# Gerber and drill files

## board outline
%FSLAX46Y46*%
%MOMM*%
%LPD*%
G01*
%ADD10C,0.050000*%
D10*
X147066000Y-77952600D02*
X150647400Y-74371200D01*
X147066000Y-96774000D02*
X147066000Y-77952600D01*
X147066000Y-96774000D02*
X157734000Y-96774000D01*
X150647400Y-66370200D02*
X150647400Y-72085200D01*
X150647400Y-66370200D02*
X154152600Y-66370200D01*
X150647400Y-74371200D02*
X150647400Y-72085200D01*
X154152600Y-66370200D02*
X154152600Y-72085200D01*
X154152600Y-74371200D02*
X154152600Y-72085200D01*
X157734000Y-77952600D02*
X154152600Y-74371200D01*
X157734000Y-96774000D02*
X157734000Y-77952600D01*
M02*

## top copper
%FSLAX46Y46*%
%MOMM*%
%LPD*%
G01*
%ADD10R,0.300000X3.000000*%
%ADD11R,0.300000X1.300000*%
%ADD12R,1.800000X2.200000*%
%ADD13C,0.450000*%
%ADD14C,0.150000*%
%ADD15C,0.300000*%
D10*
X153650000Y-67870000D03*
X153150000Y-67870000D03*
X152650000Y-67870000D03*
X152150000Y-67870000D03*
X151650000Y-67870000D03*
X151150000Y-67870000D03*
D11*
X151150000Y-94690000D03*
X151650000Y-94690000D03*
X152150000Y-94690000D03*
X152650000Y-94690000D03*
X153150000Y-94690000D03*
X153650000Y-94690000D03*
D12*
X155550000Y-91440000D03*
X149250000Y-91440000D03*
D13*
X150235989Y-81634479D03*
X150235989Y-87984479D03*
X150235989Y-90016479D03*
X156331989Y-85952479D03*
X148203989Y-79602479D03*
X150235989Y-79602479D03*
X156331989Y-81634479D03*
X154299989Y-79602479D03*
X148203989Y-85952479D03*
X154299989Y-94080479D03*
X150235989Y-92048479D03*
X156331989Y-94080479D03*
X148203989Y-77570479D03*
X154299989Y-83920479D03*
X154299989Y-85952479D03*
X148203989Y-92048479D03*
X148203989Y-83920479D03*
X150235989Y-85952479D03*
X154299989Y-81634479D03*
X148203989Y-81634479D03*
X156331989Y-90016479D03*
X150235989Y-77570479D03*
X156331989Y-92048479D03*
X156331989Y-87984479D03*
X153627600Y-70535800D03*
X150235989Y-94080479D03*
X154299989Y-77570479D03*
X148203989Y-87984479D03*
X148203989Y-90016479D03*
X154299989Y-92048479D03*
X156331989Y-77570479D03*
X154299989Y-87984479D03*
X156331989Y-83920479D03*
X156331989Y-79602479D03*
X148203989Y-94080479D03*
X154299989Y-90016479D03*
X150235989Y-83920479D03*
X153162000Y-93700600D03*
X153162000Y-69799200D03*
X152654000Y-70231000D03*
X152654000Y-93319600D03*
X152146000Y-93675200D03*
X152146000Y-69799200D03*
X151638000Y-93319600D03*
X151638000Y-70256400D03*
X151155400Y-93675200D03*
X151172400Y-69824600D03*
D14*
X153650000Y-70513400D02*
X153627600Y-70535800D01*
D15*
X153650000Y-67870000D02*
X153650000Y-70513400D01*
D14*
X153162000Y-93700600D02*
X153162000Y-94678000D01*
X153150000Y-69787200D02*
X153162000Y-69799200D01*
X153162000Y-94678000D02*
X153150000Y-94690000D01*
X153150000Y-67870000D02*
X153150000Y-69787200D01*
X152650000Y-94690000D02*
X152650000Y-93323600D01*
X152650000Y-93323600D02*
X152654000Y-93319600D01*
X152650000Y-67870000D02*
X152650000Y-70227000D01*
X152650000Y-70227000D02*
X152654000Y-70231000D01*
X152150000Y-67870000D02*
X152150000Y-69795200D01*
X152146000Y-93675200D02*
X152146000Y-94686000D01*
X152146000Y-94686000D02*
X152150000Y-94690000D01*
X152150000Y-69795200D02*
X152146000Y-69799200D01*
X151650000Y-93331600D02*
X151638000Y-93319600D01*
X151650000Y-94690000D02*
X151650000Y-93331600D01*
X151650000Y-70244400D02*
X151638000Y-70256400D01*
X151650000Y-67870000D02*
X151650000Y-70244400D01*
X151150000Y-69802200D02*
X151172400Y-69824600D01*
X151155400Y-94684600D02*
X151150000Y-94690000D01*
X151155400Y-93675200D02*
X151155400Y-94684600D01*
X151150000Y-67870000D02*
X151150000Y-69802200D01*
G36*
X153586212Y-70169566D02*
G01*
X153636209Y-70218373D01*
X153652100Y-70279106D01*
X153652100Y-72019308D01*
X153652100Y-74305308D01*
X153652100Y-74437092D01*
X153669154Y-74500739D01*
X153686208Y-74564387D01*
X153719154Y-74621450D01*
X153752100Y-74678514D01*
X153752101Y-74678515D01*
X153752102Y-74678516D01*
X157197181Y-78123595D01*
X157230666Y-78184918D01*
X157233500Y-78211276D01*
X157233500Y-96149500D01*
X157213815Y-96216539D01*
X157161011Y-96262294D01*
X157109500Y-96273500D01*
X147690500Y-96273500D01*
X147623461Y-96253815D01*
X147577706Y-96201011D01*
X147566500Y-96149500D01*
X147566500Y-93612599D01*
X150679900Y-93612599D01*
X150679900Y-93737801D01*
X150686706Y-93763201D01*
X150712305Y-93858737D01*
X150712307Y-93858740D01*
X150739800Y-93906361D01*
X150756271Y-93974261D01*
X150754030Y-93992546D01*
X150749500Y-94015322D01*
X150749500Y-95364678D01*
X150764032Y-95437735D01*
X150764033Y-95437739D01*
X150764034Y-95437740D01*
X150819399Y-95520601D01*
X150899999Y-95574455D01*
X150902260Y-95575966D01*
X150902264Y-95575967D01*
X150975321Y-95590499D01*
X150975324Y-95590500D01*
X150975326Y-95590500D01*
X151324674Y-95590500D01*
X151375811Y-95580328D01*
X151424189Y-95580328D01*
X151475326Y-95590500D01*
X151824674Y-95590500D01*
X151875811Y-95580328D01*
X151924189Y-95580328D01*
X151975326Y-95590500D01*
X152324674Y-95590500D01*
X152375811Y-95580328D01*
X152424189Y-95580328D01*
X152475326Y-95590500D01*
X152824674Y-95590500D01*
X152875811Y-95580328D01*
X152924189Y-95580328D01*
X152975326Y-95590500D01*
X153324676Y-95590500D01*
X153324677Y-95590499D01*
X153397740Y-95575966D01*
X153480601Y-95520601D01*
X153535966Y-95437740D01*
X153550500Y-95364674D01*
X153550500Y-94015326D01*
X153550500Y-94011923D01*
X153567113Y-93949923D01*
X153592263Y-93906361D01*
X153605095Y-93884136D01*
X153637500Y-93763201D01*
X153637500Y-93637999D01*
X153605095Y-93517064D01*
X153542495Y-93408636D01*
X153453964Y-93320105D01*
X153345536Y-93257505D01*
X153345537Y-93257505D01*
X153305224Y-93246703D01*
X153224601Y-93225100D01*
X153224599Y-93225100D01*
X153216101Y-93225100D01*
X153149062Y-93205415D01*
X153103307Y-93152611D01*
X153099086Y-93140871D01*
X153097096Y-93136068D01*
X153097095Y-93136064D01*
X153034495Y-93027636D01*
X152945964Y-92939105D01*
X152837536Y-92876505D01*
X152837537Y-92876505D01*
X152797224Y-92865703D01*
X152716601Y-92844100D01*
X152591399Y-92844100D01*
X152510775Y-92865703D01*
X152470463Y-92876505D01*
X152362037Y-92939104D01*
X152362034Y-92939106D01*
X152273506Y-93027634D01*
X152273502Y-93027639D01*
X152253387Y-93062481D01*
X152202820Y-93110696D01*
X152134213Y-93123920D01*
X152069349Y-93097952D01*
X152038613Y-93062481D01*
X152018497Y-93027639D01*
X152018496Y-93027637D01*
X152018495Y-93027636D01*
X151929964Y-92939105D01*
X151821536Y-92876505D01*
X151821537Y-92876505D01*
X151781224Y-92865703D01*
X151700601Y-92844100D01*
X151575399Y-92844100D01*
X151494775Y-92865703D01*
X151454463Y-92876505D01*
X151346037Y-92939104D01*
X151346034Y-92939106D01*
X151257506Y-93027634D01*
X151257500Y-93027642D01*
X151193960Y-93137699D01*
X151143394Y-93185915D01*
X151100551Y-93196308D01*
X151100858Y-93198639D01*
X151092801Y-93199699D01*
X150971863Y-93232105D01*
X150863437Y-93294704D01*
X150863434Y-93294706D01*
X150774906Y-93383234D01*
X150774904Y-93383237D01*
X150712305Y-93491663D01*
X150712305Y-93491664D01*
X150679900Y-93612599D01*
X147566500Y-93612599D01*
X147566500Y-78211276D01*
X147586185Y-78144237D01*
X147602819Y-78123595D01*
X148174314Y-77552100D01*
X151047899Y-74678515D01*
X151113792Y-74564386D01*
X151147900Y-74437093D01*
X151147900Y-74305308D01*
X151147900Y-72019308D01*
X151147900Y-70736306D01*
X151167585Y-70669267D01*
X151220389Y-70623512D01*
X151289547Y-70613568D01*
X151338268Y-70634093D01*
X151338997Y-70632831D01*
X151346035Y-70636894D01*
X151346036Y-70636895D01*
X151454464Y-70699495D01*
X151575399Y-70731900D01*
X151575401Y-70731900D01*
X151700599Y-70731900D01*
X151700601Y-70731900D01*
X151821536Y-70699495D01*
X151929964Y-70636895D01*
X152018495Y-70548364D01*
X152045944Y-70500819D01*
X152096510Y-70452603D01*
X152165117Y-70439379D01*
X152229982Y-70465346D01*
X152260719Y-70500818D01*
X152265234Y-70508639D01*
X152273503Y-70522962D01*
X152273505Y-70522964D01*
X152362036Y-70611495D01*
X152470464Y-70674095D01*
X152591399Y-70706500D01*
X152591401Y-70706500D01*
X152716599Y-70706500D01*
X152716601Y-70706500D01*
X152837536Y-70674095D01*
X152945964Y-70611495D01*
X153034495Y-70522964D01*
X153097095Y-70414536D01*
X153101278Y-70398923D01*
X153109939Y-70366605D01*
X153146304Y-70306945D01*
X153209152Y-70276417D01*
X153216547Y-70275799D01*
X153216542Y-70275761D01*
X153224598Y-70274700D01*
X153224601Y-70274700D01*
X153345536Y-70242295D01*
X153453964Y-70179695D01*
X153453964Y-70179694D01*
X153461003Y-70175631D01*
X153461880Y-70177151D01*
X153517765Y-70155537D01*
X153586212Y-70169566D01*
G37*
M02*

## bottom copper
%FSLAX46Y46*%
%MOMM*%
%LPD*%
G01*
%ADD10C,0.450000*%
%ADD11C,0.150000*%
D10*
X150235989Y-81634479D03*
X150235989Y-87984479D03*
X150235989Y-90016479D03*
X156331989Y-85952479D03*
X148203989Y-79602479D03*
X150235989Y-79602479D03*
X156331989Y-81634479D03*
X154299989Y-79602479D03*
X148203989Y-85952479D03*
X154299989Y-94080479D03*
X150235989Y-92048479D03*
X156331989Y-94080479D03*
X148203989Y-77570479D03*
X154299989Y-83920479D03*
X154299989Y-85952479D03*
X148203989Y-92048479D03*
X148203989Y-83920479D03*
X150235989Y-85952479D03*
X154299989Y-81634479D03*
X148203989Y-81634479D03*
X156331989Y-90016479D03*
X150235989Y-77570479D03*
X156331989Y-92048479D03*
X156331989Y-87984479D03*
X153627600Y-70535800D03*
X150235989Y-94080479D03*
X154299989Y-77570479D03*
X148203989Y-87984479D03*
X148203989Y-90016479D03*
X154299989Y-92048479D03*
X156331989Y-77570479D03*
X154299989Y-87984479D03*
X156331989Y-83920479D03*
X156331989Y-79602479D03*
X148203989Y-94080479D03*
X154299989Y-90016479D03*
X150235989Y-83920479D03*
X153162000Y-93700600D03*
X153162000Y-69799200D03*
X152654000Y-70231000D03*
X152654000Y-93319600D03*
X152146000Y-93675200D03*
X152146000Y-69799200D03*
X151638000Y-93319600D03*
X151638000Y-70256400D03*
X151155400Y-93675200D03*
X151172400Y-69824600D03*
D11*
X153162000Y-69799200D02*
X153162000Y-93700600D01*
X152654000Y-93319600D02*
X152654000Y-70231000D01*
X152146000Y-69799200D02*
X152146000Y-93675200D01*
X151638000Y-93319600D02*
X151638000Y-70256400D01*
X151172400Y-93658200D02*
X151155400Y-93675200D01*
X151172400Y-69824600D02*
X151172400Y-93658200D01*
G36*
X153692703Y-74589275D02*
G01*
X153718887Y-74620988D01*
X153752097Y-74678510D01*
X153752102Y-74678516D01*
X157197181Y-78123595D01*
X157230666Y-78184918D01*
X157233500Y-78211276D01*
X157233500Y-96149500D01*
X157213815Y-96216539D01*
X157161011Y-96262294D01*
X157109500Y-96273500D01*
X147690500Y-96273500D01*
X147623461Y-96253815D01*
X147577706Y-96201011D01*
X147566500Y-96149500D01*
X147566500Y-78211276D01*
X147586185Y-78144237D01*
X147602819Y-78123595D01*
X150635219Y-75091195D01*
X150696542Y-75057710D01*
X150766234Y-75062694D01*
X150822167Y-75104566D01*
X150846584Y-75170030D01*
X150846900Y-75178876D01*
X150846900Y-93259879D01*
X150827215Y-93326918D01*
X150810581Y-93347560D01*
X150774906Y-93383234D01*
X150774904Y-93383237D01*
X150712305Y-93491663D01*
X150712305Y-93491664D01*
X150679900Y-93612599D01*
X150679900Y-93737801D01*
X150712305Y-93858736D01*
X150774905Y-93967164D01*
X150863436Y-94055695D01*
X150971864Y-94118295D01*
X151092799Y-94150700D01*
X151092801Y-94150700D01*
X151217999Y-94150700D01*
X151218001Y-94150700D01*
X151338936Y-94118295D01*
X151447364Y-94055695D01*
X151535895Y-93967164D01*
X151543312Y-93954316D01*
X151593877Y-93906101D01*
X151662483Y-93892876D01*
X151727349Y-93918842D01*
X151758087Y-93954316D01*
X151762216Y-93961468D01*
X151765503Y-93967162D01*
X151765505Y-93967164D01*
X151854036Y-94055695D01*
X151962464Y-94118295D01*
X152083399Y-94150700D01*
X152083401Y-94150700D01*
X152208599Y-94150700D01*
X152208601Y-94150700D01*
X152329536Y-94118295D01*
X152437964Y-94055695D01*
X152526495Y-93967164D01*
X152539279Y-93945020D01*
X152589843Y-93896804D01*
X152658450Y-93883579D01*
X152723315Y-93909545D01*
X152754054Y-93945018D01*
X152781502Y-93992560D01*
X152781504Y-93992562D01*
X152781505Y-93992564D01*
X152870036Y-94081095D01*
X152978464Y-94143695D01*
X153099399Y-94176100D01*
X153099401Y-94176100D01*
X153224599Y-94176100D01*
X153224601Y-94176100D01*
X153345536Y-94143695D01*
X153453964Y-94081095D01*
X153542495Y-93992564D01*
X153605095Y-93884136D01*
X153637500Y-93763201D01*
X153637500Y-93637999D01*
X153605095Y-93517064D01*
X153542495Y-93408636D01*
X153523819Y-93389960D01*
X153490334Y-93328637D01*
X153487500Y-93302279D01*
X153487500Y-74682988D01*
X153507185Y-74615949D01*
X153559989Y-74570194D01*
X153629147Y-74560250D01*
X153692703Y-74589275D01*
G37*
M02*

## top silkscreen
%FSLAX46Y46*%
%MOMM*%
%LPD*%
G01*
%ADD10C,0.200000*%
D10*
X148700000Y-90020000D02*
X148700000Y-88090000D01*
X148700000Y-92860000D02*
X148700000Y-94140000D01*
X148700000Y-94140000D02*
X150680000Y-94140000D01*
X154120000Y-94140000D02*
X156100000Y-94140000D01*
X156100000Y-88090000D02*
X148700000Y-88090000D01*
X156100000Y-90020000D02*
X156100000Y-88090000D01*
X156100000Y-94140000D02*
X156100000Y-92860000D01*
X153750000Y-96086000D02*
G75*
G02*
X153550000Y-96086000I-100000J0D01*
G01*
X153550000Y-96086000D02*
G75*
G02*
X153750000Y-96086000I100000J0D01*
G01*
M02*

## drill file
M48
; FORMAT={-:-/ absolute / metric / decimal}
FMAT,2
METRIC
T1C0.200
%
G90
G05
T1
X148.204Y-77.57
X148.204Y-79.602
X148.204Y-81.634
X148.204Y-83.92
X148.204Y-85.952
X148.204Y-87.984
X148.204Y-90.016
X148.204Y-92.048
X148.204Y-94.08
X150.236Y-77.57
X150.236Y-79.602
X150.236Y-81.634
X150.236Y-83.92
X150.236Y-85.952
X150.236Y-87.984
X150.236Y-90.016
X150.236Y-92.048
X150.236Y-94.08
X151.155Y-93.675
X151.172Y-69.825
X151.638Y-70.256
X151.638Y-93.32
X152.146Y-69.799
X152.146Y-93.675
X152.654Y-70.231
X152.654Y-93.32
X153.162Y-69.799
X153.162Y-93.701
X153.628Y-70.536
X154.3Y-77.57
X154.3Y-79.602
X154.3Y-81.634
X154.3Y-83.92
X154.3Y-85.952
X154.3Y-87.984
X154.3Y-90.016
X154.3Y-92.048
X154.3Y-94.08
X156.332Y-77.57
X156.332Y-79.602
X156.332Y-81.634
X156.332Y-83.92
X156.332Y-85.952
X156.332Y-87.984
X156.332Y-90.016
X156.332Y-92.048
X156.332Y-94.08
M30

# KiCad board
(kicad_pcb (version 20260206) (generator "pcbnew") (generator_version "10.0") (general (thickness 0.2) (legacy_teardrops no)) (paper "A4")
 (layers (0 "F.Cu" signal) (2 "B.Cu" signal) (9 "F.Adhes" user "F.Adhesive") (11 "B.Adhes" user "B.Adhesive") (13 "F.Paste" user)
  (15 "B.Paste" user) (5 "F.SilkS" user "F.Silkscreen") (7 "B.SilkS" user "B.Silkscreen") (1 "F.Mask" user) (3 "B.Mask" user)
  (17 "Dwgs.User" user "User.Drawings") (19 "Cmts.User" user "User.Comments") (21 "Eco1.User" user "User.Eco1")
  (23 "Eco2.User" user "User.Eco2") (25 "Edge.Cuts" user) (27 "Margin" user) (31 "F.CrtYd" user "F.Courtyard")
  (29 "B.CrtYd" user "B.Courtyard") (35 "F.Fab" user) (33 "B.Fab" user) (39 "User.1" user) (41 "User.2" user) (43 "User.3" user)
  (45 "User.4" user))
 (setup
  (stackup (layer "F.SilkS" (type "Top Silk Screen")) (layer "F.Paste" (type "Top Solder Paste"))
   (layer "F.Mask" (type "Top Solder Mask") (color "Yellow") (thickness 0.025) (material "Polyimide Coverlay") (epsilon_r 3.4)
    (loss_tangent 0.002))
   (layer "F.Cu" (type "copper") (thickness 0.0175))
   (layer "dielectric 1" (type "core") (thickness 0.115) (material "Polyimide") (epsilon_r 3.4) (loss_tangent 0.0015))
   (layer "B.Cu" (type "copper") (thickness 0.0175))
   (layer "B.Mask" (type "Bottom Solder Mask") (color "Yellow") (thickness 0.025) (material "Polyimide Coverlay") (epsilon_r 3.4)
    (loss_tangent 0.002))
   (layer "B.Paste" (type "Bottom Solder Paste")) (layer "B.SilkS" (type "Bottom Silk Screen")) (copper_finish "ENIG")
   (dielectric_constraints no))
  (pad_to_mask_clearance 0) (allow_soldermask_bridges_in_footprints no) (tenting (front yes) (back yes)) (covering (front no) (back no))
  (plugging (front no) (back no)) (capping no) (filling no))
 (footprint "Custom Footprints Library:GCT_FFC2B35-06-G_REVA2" (layer "F.Cu") (at 152.4 71.12)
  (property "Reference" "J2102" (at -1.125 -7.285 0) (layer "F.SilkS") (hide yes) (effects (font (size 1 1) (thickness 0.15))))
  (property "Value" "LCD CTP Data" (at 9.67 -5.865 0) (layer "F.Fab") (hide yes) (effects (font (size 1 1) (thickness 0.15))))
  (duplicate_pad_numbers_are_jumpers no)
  (pad "1" smd rect (at 1.25 -3.25) (size 0.3 3) (layers "F.Cu" "F.Mask" "F.Paste") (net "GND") (solder_mask_margin 0.102))
  (pad "2" smd rect (at 0.75 -3.25) (size 0.3 3) (layers "F.Cu" "F.Mask" "F.Paste") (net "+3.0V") (solder_mask_margin 0.102))
  (pad "3" smd rect (at 0.25 -3.25) (size 0.3 3) (layers "F.Cu" "F.Mask" "F.Paste") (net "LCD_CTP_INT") (solder_mask_margin 0.102))
  (pad "4" smd rect (at -0.25 -3.25) (size 0.3 3) (layers "F.Cu" "F.Mask" "F.Paste") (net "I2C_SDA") (solder_mask_margin 0.102))
  (pad "5" smd rect (at -0.75 -3.25) (size 0.3 3) (layers "F.Cu" "F.Mask" "F.Paste") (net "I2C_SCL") (solder_mask_margin 0.102))
  (pad "6" smd rect (at -1.25 -3.25) (size 0.3 3) (layers "F.Cu" "F.Mask" "F.Paste") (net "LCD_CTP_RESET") (solder_mask_margin 0.102)))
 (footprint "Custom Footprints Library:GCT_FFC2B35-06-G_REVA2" (layer "F.Cu") (at 152.4 91.44 180)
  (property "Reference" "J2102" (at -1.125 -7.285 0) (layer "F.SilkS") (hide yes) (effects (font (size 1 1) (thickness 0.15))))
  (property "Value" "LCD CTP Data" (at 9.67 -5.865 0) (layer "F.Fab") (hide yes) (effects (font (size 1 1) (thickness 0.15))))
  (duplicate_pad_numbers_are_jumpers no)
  (fp_line (start 3.7 1.42) (end 3.7 3.35) (stroke (width 0.2) (type solid)) (layer "F.SilkS"))
  (fp_line (start 3.7 -1.42) (end 3.7 -2.7) (stroke (width 0.2) (type solid)) (layer "F.SilkS"))
  (fp_line (start 3.7 -2.7) (end 1.72 -2.7) (stroke (width 0.2) (type solid)) (layer "F.SilkS"))
  (fp_line (start -1.72 -2.7) (end -3.7 -2.7) (stroke (width 0.2) (type solid)) (layer "F.SilkS"))
  (fp_line (start -3.7 3.35) (end 3.7 3.35) (stroke (width 0.2) (type solid)) (layer "F.SilkS"))
  (fp_line (start -3.7 1.42) (end -3.7 3.35) (stroke (width 0.2) (type solid)) (layer "F.SilkS"))
  (fp_line (start -3.7 -2.7) (end -3.7 -1.42) (stroke (width 0.2) (type solid)) (layer "F.SilkS"))
  (fp_circle (center -1.25 -4.646) (end -1.15 -4.646) (stroke (width 0.2) (type solid)) (fill no) (layer "F.SilkS"))
  (pad "1" smd rect (at 1.25 -3.25 180) (size 0.3 1.3) (layers "F.Cu" "F.Mask" "F.Paste") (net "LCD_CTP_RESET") (solder_mask_margin 0.102))
  (pad "2" smd rect (at 0.75 -3.25 180) (size 0.3 1.3) (layers "F.Cu" "F.Mask" "F.Paste") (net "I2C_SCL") (solder_mask_margin 0.102))
  (pad "3" smd rect (at 0.25 -3.25 180) (size 0.3 1.3) (layers "F.Cu" "F.Mask" "F.Paste") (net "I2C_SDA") (solder_mask_margin 0.102))
  (pad "4" smd rect (at -0.25 -3.25 180) (size 0.3 1.3) (layers "F.Cu" "F.Mask" "F.Paste") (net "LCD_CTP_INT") (solder_mask_margin 0.102))
  (pad "5" smd rect (at -0.75 -3.25 180) (size 0.3 1.3) (layers "F.Cu" "F.Mask" "F.Paste") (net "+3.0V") (solder_mask_margin 0.102))
  (pad "6" smd rect (at -1.25 -3.25 180) (size 0.3 1.3) (layers "F.Cu" "F.Mask" "F.Paste") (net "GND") (solder_mask_margin 0.102)
   (zone_connect 2))
  (pad "S1" smd rect (at -3.15 0 180) (size 1.8 2.2) (layers "F.Cu" "F.Mask" "F.Paste") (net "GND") (solder_mask_margin 0.102))
  (pad "S2" smd rect (at 3.15 0 180) (size 1.8 2.2) (layers "F.Cu" "F.Mask" "F.Paste") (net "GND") (solder_mask_margin 0.102)))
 (gr_line (start 147.066 77.9526) (end 150.6474 74.3712) (stroke (width 0.05) (type default)) (layer "Edge.Cuts"))
 (gr_line (start 147.066 96.774) (end 147.066 77.9526) (stroke (width 0.05) (type default)) (layer "Edge.Cuts"))
 (gr_line (start 147.066 96.774) (end 157.734 96.774) (stroke (width 0.05) (type default)) (layer "Edge.Cuts"))
 (gr_line (start 150.6474 66.3702) (end 150.6474 72.0852) (stroke (width 0.05) (type default)) (layer "Edge.Cuts"))
 (gr_line (start 150.6474 66.3702) (end 154.1526 66.3702) (stroke (width 0.05) (type default)) (layer "Edge.Cuts"))
 (gr_line (start 150.6474 74.3712) (end 150.6474 72.0852) (stroke (width 0.05) (type default)) (layer "Edge.Cuts"))
 (gr_line (start 154.1526 66.3702) (end 154.1526 72.0852) (stroke (width 0.05) (type default)) (layer "Edge.Cuts"))
 (gr_line (start 154.1526 74.3712) (end 154.1526 72.0852) (stroke (width 0.05) (type default)) (layer "Edge.Cuts"))
 (gr_line (start 157.734 77.9526) (end 154.1526 74.3712) (stroke (width 0.05) (type default)) (layer "Edge.Cuts"))
 (gr_line (start 157.734 96.774) (end 157.734 77.9526) (stroke (width 0.05) (type default)) (layer "Edge.Cuts"))
 (segment (start 153.65 70.5134) (end 153.6276 70.5358) (width 0.15) (layer "F.Cu") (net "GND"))
 (segment (start 153.65 67.87) (end 153.65 70.5134) (width 0.3) (layer "F.Cu") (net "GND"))
 (via (at 150.235989 81.634479) (size 0.45) (drill 0.2) (layers "F.Cu" "B.Cu") (free yes) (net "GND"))
 (via (at 150.235989 87.984479) (size 0.45) (drill 0.2) (layers "F.Cu" "B.Cu") (free yes) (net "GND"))
 (via (at 150.235989 90.016479) (size 0.45) (drill 0.2) (layers "F.Cu" "B.Cu") (free yes) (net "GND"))
 (via (at 156.331989 85.952479) (size 0.45) (drill 0.2) (layers "F.Cu" "B.Cu") (free yes) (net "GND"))
 (via (at 148.203989 79.602479) (size 0.45) (drill 0.2) (layers "F.Cu" "B.Cu") (free yes) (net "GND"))
 (via (at 150.235989 79.602479) (size 0.45) (drill 0.2) (layers "F.Cu" "B.Cu") (free yes) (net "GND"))
 (via (at 156.331989 81.634479) (size 0.45) (drill 0.2) (layers "F.Cu" "B.Cu") (free yes) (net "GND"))
 (via (at 154.299989 79.602479) (size 0.45) (drill 0.2) (layers "F.Cu" "B.Cu") (free yes) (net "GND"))
 (via (at 148.203989 85.952479) (size 0.45) (drill 0.2) (layers "F.Cu" "B.Cu") (free yes) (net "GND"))
 (via (at 154.299989 94.080479) (size 0.45) (drill 0.2) (layers "F.Cu" "B.Cu") (free yes) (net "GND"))
 (via (at 150.235989 92.048479) (size 0.45) (drill 0.2) (layers "F.Cu" "B.Cu") (free yes) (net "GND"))
 (via (at 156.331989 94.080479) (size 0.45) (drill 0.2) (layers "F.Cu" "B.Cu") (free yes) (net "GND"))
 (via (at 148.203989 77.570479) (size 0.45) (drill 0.2) (layers "F.Cu" "B.Cu") (free yes) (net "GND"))
 (via (at 154.299989 83.920479) (size 0.45) (drill 0.2) (layers "F.Cu" "B.Cu") (free yes) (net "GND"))
 (via (at 154.299989 85.952479) (size 0.45) (drill 0.2) (layers "F.Cu" "B.Cu") (free yes) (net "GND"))
 (via (at 148.203989 92.048479) (size 0.45) (drill 0.2) (layers "F.Cu" "B.Cu") (free yes) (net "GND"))
 (via (at 148.203989 83.920479) (size 0.45) (drill 0.2) (layers "F.Cu" "B.Cu") (free yes) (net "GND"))
 (via (at 150.235989 85.952479) (size 0.45) (drill 0.2) (layers "F.Cu" "B.Cu") (free yes) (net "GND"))
 (via (at 154.299989 81.634479) (size 0.45) (drill 0.2) (layers "F.Cu" "B.Cu") (free yes) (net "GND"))
 (via (at 148.203989 81.634479) (size 0.45) (drill 0.2) (layers "F.Cu" "B.Cu") (free yes) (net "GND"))
 (via (at 156.331989 90.016479) (size 0.45) (drill 0.2) (layers "F.Cu" "B.Cu") (free yes) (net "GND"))
 (via (at 150.235989 77.570479) (size 0.45) (drill 0.2) (layers "F.Cu" "B.Cu") (free yes) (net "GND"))
 (via (at 156.331989 92.048479) (size 0.45) (drill 0.2) (layers "F.Cu" "B.Cu") (free yes) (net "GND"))
 (via (at 156.331989 87.984479) (size 0.45) (drill 0.2) (layers "F.Cu" "B.Cu") (free yes) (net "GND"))
 (via (at 153.6276 70.5358) (size 0.45) (drill 0.2) (layers "F.Cu" "B.Cu") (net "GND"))
 (via (at 150.235989 94.080479) (size 0.45) (drill 0.2) (layers "F.Cu" "B.Cu") (free yes) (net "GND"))
 (via (at 154.299989 77.570479) (size 0.45) (drill 0.2) (layers "F.Cu" "B.Cu") (free yes) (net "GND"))
 (via (at 148.203989 87.984479) (size 0.45) (drill 0.2) (layers "F.Cu" "B.Cu") (free yes) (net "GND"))
 (via (at 148.203989 90.016479) (size 0.45) (drill 0.2) (layers "F.Cu" "B.Cu") (free yes) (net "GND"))
 (via (at 154.299989 92.048479) (size 0.45) (drill 0.2) (layers "F.Cu" "B.Cu") (free yes) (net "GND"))
 (via (at 156.331989 77.570479) (size 0.45) (drill 0.2) (layers "F.Cu" "B.Cu") (free yes) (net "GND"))
 (via (at 154.299989 87.984479) (size 0.45) (drill 0.2) (layers "F.Cu" "B.Cu") (free yes) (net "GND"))
 (via (at 156.331989 83.920479) (size 0.45) (drill 0.2) (layers "F.Cu" "B.Cu") (free yes) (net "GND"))
 (via (at 156.331989 79.602479) (size 0.45) (drill 0.2) (layers "F.Cu" "B.Cu") (free yes) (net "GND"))
 (via (at 148.203989 94.080479) (size 0.45) (drill 0.2) (layers "F.Cu" "B.Cu") (free yes) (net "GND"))
 (via (at 154.299989 90.016479) (size 0.45) (drill 0.2) (layers "F.Cu" "B.Cu") (free yes) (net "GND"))
 (via (at 150.235989 83.920479) (size 0.45) (drill 0.2) (layers "F.Cu" "B.Cu") (free yes) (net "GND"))
 (segment (start 153.162 93.7006) (end 153.162 94.678) (width 0.15) (layer "F.Cu") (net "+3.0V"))
 (segment (start 153.15 69.7872) (end 153.162 69.7992) (width 0.15) (layer "F.Cu") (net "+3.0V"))
 (segment (start 153.162 94.678) (end 153.15 94.69) (width 0.15) (layer "F.Cu") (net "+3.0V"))
 (segment (start 153.15 67.87) (end 153.15 69.7872) (width 0.15) (layer "F.Cu") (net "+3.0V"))
 (via (at 153.162 93.7006) (size 0.45) (drill 0.2) (layers "F.Cu" "B.Cu") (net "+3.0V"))
 (via (at 153.162 69.7992) (size 0.45) (drill 0.2) (layers "F.Cu" "B.Cu") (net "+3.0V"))
 (segment (start 153.162 69.7992) (end 153.162 93.7006) (width 0.15) (layer "B.Cu") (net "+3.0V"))
 (segment (start 152.65 94.69) (end 152.65 93.3236) (width 0.15) (layer "F.Cu") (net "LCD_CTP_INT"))
 (segment (start 152.65 93.3236) (end 152.654 93.3196) (width 0.15) (layer "F.Cu") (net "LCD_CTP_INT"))
 (segment (start 152.65 67.87) (end 152.65 70.227) (width 0.15) (layer "F.Cu") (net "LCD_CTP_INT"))
 (segment (start 152.65 70.227) (end 152.654 70.231) (width 0.15) (layer "F.Cu") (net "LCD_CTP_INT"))
 (via (at 152.654 70.231) (size 0.45) (drill 0.2) (layers "F.Cu" "B.Cu") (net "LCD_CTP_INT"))
 (via (at 152.654 93.3196) (size 0.45) (drill 0.2) (layers "F.Cu" "B.Cu") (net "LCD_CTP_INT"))
 (segment (start 152.654 93.3196) (end 152.654 70.231) (width 0.15) (layer "B.Cu") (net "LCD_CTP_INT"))
 (segment (start 152.15 67.87) (end 152.15 69.7952) (width 0.15) (layer "F.Cu") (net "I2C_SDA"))
 (segment (start 152.146 93.6752) (end 152.146 94.686) (width 0.15) (layer "F.Cu") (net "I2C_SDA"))
 (segment (start 152.146 94.686) (end 152.15 94.69) (width 0.15) (layer "F.Cu") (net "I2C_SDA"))
 (segment (start 152.15 69.7952) (end 152.146 69.7992) (width 0.15) (layer "F.Cu") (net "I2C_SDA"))
 (via (at 152.146 93.6752) (size 0.45) (drill 0.2) (layers "F.Cu" "B.Cu") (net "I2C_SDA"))
 (via (at 152.146 69.7992) (size 0.45) (drill 0.2) (layers "F.Cu" "B.Cu") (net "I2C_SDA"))
 (segment (start 152.146 69.7992) (end 152.146 93.6752) (width 0.15) (layer "B.Cu") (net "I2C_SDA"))
 (segment (start 151.65 93.3316) (end 151.638 93.3196) (width 0.15) (layer "F.Cu") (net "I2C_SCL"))
 (segment (start 151.65 94.69) (end 151.65 93.3316) (width 0.15) (layer "F.Cu") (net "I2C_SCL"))
 (segment (start 151.65 70.2444) (end 151.638 70.2564) (width 0.15) (layer "F.Cu") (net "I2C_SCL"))
 (segment (start 151.65 67.87) (end 151.65 70.2444) (width 0.15) (layer "F.Cu") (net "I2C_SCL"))
 (via (at 151.638 93.3196) (size 0.45) (drill 0.2) (layers "F.Cu" "B.Cu") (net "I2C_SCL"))
 (via (at 151.638 70.2564) (size 0.45) (drill 0.2) (layers "F.Cu" "B.Cu") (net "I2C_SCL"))
 (segment (start 151.638 93.3196) (end 151.638 70.2564) (width 0.15) (layer "B.Cu") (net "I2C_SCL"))
 (segment (start 151.15 69.8022) (end 151.1724 69.8246) (width 0.15) (layer "F.Cu") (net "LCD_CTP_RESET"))
 (segment (start 151.1554 94.6846) (end 151.15 94.69) (width 0.15) (layer "F.Cu") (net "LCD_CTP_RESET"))
 (segment (start 151.1554 93.6752) (end 151.1554 94.6846) (width 0.15) (layer "F.Cu") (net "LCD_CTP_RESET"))
 (segment (start 151.15 67.87) (end 151.15 69.8022) (width 0.15) (layer "F.Cu") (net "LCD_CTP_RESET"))
 (via (at 151.1554 93.6752) (size 0.45) (drill 0.2) (layers "F.Cu" "B.Cu") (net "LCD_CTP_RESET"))
 (via (at 151.1724 69.8246) (size 0.45) (drill 0.2) (layers "F.Cu" "B.Cu") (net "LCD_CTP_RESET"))
 (segment (start 151.1724 93.6582) (end 151.1554 93.6752) (width 0.15) (layer "B.Cu") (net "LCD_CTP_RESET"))
 (segment (start 151.1724 69.8246) (end 151.1724 93.6582) (width 0.15) (layer "B.Cu") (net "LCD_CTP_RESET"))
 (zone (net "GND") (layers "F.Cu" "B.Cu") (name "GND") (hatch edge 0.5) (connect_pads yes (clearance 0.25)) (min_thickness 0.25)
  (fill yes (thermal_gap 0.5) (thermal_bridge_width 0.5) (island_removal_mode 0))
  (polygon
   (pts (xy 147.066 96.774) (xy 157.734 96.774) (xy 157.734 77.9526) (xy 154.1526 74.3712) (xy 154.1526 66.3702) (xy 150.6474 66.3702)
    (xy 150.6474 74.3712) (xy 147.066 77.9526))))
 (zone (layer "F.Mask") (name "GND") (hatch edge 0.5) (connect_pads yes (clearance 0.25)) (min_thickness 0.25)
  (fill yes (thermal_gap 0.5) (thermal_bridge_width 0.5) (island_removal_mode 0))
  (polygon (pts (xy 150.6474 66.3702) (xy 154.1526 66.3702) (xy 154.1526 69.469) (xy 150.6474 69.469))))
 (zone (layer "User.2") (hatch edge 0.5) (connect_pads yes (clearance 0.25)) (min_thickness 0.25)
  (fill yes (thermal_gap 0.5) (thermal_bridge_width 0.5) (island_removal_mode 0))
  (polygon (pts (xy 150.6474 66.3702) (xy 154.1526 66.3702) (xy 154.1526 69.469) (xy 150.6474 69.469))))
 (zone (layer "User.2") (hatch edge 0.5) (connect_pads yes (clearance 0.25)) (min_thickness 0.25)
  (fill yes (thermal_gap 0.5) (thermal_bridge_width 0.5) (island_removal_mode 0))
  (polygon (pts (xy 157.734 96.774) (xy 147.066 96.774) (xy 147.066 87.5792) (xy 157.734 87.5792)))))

